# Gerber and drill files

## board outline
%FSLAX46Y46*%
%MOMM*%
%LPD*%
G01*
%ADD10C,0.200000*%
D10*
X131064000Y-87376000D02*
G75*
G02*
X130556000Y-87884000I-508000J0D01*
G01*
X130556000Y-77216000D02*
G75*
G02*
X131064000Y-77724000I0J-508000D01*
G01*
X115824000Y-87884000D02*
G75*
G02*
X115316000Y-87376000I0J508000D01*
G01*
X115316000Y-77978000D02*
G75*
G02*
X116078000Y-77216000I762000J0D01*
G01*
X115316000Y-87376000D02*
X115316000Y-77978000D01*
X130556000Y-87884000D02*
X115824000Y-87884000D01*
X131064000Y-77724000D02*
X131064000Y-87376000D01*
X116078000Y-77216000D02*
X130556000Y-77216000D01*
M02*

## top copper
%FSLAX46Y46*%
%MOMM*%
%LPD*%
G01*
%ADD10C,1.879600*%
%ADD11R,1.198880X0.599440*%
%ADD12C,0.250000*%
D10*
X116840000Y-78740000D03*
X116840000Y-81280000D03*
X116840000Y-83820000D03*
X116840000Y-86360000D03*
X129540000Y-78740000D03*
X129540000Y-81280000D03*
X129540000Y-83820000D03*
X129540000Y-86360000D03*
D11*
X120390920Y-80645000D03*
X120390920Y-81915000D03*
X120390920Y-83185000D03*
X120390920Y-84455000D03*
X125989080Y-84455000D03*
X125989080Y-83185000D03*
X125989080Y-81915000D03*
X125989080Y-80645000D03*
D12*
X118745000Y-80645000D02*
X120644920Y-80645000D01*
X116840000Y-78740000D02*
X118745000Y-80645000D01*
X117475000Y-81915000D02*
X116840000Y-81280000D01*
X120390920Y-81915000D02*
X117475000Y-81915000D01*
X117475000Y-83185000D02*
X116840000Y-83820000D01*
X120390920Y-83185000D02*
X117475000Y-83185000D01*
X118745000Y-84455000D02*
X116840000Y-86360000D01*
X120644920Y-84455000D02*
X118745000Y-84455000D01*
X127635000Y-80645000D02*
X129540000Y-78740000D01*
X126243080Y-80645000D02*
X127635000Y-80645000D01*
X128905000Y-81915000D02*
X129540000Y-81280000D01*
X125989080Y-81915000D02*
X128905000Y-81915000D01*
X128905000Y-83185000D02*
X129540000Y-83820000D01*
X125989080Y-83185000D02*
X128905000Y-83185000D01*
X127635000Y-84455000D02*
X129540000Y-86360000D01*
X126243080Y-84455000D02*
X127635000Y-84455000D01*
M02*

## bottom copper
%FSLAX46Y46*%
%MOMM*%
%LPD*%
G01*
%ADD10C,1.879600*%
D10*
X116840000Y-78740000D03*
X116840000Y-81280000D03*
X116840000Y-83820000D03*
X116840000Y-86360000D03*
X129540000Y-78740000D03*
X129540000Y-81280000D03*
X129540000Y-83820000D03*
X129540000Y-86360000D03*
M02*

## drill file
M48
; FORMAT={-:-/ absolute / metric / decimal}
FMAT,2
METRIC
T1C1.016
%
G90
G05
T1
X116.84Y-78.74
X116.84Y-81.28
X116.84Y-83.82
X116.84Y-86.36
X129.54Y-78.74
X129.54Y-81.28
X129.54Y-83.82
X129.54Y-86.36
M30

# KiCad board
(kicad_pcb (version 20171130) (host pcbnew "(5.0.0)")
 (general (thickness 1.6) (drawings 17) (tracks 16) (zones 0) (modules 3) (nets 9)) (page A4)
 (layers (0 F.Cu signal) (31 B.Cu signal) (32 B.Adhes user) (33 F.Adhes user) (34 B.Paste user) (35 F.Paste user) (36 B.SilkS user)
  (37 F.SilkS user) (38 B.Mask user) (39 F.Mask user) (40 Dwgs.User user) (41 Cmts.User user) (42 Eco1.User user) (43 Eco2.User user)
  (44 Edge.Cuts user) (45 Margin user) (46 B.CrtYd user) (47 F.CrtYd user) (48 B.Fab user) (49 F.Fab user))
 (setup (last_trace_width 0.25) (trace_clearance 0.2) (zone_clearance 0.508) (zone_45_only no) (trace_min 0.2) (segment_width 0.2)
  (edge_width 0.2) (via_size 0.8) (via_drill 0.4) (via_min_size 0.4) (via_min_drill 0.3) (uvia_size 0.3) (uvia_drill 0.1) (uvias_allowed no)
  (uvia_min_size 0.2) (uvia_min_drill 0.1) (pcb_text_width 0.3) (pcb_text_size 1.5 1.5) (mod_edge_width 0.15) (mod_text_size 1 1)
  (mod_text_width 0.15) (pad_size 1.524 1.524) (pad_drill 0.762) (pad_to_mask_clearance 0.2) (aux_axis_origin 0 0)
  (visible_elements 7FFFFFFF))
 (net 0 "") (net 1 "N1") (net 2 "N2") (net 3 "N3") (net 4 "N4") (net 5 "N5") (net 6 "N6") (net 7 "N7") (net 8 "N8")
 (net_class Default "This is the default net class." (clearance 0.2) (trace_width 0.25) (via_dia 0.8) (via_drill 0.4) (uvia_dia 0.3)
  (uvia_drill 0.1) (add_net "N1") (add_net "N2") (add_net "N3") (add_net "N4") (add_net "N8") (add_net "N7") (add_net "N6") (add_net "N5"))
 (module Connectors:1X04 (layer F.Cu) (at 116.84 78.74 270)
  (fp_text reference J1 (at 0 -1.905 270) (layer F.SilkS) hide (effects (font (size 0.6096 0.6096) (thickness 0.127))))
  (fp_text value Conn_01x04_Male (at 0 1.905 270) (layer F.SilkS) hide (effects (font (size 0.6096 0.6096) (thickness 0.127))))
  (pad 1 thru_hole circle (at 0 0 270) (size 1.8796 1.8796) (drill 1.016) (layers *.Cu *.Mask) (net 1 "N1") (solder_mask_margin 0.1016))
  (pad 2 thru_hole circle (at 2.54 0 270) (size 1.8796 1.8796) (drill 1.016) (layers *.Cu *.Mask) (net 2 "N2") (solder_mask_margin 0.1016))
  (pad 3 thru_hole circle (at 5.08 0 270) (size 1.8796 1.8796) (drill 1.016) (layers *.Cu *.Mask) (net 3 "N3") (solder_mask_margin 0.1016))
  (pad 4 thru_hole circle (at 7.62 0 270) (size 1.8796 1.8796) (drill 1.016) (layers *.Cu *.Mask) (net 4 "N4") (solder_mask_margin 0.1016)))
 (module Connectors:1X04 (layer F.Cu) (at 129.54 86.36 90)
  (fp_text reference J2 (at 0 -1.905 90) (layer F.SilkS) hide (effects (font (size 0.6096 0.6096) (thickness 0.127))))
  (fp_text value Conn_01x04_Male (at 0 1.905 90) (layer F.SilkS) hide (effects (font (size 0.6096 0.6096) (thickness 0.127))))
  (pad 4 thru_hole circle (at 7.62 0 90) (size 1.8796 1.8796) (drill 1.016) (layers *.Cu *.Mask) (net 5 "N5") (solder_mask_margin 0.1016))
  (pad 3 thru_hole circle (at 5.08 0 90) (size 1.8796 1.8796) (drill 1.016) (layers *.Cu *.Mask) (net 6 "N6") (solder_mask_margin 0.1016))
  (pad 2 thru_hole circle (at 2.54 0 90) (size 1.8796 1.8796) (drill 1.016) (layers *.Cu *.Mask) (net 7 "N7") (solder_mask_margin 0.1016))
  (pad 1 thru_hole circle (at 0 0 90) (size 1.8796 1.8796) (drill 1.016) (layers *.Cu *.Mask) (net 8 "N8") (solder_mask_margin 0.1016)))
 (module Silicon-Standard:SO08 (layer F.Cu) (at 123.19 82.55 270)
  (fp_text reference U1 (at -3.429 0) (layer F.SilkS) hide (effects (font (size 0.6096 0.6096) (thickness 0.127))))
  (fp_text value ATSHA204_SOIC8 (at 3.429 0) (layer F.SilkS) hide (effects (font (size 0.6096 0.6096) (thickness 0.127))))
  (pad 1 smd rect (at -1.905 2.79908 270) (size 0.59944 1.19888) (layers F.Cu F.Paste F.Mask) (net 1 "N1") (solder_mask_margin 0.1016))
  (pad 2 smd rect (at -0.635 2.79908 270) (size 0.59944 1.19888) (layers F.Cu F.Paste F.Mask) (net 2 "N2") (solder_mask_margin 0.1016))
  (pad 3 smd rect (at 0.635 2.79908 270) (size 0.59944 1.19888) (layers F.Cu F.Paste F.Mask) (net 3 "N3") (solder_mask_margin 0.1016))
  (pad 4 smd rect (at 1.905 2.79908 270) (size 0.59944 1.19888) (layers F.Cu F.Paste F.Mask) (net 4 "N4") (solder_mask_margin 0.1016))
  (pad 5 smd rect (at 1.905 -2.79908 270) (size 0.59944 1.19888) (layers F.Cu F.Paste F.Mask) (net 8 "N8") (solder_mask_margin 0.1016))
  (pad 6 smd rect (at 0.635 -2.79908 270) (size 0.59944 1.19888) (layers F.Cu F.Paste F.Mask) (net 7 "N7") (solder_mask_margin 0.1016))
  (pad 7 smd rect (at -0.635 -2.79908 270) (size 0.59944 1.19888) (layers F.Cu F.Paste F.Mask) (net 6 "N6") (solder_mask_margin 0.1016))
  (pad 8 smd rect (at -1.905 -2.79908 270) (size 0.59944 1.19888) (layers F.Cu F.Paste F.Mask) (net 5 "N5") (solder_mask_margin 0.1016)))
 (gr_arc (start 130.556 87.376) (end 130.556 87.884) (angle -90) (layer Edge.Cuts) (width 0.2))
 (gr_arc (start 130.556 77.724) (end 131.064 77.724) (angle -90) (layer Edge.Cuts) (width 0.2))
 (gr_arc (start 115.824 87.376) (end 115.316 87.376) (angle -90) (layer Edge.Cuts) (width 0.2))
 (gr_arc (start 116.078 77.978) (end 116.078 77.216) (angle -90) (layer Edge.Cuts) (width 0.2))
 (gr_line (start 115.316 87.376) (end 115.316 77.978) (layer Edge.Cuts) (width 0.2))
 (gr_line (start 130.556 87.884) (end 115.824 87.884) (layer Edge.Cuts) (width 0.2))
 (gr_line (start 131.064 77.724) (end 131.064 87.376) (layer Edge.Cuts) (width 0.2))
 (gr_line (start 116.078 77.216) (end 130.556 77.216) (layer Edge.Cuts) (width 0.2))
 (segment (start 118.745 80.645) (end 120.64492 80.645) (width 0.25) (layer F.Cu) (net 1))
 (segment (start 116.84 78.74) (end 118.745 80.645) (width 0.25) (layer F.Cu) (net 1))
 (segment (start 117.475 81.915) (end 116.84 81.28) (width 0.25) (layer F.Cu) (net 2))
 (segment (start 120.39092 81.915) (end 117.475 81.915) (width 0.25) (layer F.Cu) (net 2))
 (segment (start 117.475 83.185) (end 116.84 83.82) (width 0.25) (layer F.Cu) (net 3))
 (segment (start 120.39092 83.185) (end 117.475 83.185) (width 0.25) (layer F.Cu) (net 3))
 (segment (start 118.745 84.455) (end 116.84 86.36) (width 0.25) (layer F.Cu) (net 4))
 (segment (start 120.64492 84.455) (end 118.745 84.455) (width 0.25) (layer F.Cu) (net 4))
 (segment (start 127.635 80.645) (end 129.54 78.74) (width 0.25) (layer F.Cu) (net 5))
 (segment (start 126.24308 80.645) (end 127.635 80.645) (width 0.25) (layer F.Cu) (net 5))
 (segment (start 128.905 81.915) (end 129.54 81.28) (width 0.25) (layer F.Cu) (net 6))
 (segment (start 125.98908 81.915) (end 128.905 81.915) (width 0.25) (layer F.Cu) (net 6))
 (segment (start 128.905 83.185) (end 129.54 83.82) (width 0.25) (layer F.Cu) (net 7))
 (segment (start 125.98908 83.185) (end 128.905 83.185) (width 0.25) (layer F.Cu) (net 7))
 (segment (start 127.635 84.455) (end 129.54 86.36) (width 0.25) (layer F.Cu) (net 8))
 (segment (start 126.24308 84.455) (end 127.635 84.455) (width 0.25) (layer F.Cu) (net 8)))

